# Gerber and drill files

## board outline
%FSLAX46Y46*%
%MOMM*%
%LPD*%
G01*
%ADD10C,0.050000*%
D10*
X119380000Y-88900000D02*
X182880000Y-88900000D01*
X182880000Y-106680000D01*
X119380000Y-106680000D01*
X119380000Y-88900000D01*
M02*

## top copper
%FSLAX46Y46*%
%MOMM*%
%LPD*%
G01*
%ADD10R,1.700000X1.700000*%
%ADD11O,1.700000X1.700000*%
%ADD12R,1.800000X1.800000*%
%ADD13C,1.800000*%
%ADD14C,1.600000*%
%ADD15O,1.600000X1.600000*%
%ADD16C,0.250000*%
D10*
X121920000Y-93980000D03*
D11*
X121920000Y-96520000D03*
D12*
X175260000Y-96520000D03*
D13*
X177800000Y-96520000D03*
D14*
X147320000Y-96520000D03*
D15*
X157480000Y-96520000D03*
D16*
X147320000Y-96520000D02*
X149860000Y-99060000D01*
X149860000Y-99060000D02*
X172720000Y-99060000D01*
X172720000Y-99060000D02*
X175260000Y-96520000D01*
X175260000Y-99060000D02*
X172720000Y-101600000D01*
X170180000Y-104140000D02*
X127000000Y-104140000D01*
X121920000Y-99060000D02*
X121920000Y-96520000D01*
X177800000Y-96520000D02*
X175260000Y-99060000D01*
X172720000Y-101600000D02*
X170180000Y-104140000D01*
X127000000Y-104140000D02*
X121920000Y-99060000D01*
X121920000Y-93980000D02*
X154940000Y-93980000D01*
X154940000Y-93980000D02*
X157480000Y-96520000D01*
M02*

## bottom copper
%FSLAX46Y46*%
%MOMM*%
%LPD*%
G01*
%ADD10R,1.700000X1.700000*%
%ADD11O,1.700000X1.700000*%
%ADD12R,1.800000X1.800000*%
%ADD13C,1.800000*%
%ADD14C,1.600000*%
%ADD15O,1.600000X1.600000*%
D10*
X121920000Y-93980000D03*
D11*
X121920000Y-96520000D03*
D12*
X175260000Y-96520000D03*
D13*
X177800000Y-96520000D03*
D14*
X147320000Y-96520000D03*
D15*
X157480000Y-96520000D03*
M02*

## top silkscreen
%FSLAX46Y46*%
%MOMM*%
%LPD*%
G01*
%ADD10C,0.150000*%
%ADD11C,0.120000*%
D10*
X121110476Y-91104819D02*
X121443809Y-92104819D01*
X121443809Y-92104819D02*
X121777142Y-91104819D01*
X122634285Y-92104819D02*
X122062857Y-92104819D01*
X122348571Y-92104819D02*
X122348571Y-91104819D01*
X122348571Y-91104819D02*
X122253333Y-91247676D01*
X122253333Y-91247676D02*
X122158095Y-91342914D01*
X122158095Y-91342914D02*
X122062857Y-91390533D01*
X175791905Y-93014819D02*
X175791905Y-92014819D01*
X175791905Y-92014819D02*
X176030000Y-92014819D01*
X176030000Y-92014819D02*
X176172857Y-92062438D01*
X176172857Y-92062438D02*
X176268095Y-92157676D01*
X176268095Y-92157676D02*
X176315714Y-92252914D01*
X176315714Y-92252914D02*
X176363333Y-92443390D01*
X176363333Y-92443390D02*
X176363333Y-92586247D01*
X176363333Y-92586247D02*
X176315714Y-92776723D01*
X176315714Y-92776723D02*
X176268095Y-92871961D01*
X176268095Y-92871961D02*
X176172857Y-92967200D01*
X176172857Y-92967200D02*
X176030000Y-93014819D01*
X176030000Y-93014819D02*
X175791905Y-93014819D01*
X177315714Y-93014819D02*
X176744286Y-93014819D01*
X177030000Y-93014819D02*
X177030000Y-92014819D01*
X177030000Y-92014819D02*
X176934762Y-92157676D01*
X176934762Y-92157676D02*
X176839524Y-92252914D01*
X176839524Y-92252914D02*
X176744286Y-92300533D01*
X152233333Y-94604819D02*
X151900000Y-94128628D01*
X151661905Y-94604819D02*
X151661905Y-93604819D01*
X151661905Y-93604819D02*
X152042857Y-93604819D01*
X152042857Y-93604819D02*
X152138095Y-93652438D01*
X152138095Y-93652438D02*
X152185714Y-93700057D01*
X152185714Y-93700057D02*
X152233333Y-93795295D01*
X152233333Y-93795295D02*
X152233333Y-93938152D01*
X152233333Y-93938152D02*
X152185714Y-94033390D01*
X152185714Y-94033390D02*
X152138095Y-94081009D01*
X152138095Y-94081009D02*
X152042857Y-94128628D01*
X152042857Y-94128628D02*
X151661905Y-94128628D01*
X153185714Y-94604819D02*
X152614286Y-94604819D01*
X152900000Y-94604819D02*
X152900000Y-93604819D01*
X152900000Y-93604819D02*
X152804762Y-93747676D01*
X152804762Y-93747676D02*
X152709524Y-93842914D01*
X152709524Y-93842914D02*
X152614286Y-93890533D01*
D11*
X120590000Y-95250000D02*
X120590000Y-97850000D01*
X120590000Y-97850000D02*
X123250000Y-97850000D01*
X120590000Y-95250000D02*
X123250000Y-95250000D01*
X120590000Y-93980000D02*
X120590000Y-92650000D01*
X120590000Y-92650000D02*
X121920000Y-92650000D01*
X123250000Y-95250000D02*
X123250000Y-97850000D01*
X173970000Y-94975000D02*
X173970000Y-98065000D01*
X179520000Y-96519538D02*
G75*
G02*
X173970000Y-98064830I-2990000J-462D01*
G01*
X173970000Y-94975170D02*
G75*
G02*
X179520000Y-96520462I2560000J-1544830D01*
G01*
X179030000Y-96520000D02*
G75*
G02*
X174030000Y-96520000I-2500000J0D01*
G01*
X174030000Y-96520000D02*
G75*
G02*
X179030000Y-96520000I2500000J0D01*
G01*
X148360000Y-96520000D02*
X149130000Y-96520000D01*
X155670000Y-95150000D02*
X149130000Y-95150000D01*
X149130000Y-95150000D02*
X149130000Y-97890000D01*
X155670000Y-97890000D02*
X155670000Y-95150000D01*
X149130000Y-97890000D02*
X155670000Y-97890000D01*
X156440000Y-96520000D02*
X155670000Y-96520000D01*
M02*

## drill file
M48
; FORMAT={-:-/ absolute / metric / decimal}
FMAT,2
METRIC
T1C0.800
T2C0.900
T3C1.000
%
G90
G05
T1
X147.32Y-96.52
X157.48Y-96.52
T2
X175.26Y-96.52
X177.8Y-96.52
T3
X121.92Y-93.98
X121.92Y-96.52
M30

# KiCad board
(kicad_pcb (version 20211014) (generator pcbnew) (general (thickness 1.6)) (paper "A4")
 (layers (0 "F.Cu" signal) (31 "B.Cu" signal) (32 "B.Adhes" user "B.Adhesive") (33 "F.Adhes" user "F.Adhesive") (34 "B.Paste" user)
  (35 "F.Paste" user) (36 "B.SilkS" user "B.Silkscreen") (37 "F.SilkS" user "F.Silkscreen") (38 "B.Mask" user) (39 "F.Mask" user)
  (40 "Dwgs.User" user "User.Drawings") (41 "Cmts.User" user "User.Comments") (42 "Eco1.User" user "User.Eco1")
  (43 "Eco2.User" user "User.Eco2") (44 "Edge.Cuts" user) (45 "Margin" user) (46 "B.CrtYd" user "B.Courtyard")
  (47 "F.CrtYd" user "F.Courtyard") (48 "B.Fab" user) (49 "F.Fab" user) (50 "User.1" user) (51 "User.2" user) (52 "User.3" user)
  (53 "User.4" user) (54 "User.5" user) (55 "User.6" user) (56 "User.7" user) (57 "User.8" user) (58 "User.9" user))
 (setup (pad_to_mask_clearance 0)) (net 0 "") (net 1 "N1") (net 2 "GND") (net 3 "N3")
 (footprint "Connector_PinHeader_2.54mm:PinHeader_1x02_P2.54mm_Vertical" (layer "F.Cu") (at 121.92 93.98)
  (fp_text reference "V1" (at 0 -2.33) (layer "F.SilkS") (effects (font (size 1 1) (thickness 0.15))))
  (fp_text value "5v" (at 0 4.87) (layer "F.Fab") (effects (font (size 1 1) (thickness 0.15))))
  (fp_line (start -1.33 1.27) (end -1.33 3.87) (layer "F.SilkS") (width 0.12))
  (fp_line (start -1.33 3.87) (end 1.33 3.87) (layer "F.SilkS") (width 0.12))
  (fp_line (start -1.33 1.27) (end 1.33 1.27) (layer "F.SilkS") (width 0.12))
  (fp_line (start -1.33 0) (end -1.33 -1.33) (layer "F.SilkS") (width 0.12))
  (fp_line (start -1.33 -1.33) (end 0 -1.33) (layer "F.SilkS") (width 0.12))
  (fp_line (start 1.33 1.27) (end 1.33 3.87) (layer "F.SilkS") (width 0.12))
  (pad "1" thru_hole rect (at 0 0) (size 1.7 1.7) (drill 1) (layers *.Cu *.Mask) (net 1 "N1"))
  (pad "2" thru_hole oval (at 0 2.54) (size 1.7 1.7) (drill 1) (layers *.Cu *.Mask) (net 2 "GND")))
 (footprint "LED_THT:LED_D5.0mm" (layer "F.Cu") (at 175.26 96.52)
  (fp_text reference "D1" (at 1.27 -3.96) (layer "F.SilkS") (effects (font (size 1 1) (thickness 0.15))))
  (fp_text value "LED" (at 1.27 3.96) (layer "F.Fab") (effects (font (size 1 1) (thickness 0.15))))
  (fp_line (start -1.29 -1.545) (end -1.29 1.545) (layer "F.SilkS") (width 0.12))
  (fp_arc (start 4.26 -0.000462) (mid 2.072002 2.880433) (end -1.29 1.54483) (layer "F.SilkS") (width 0.12))
  (fp_arc (start -1.29 -1.54483) (mid 2.072002 -2.880433) (end 4.26 0.000462) (layer "F.SilkS") (width 0.12))
  (fp_circle (center 1.27 0) (end 3.77 0) (layer "F.SilkS") (width 0.12) (fill none))
  (pad "1" thru_hole rect (at 0 0) (size 1.8 1.8) (drill 0.9) (layers *.Cu *.Mask) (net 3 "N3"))
  (pad "2" thru_hole circle (at 2.54 0) (size 1.8 1.8) (drill 0.9) (layers *.Cu *.Mask) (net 2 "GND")))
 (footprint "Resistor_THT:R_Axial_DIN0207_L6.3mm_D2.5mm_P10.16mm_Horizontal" (layer "F.Cu") (at 147.32 96.52)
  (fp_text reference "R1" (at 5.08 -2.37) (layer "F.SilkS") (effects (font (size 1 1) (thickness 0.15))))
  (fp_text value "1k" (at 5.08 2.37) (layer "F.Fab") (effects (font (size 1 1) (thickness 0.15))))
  (fp_line (start 1.04 0) (end 1.81 0) (layer "F.SilkS") (width 0.12))
  (fp_line (start 8.35 -1.37) (end 1.81 -1.37) (layer "F.SilkS") (width 0.12))
  (fp_line (start 1.81 -1.37) (end 1.81 1.37) (layer "F.SilkS") (width 0.12))
  (fp_line (start 8.35 1.37) (end 8.35 -1.37) (layer "F.SilkS") (width 0.12))
  (fp_line (start 1.81 1.37) (end 8.35 1.37) (layer "F.SilkS") (width 0.12))
  (fp_line (start 9.12 0) (end 8.35 0) (layer "F.SilkS") (width 0.12))
  (pad "1" thru_hole circle (at 0 0) (size 1.6 1.6) (drill 0.8) (layers *.Cu *.Mask) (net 3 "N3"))
  (pad "2" thru_hole oval (at 10.16 0) (size 1.6 1.6) (drill 0.8) (layers *.Cu *.Mask) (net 1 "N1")))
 (gr_rect (start 119.38 88.9) (end 182.88 106.68) (layer "Edge.Cuts") (width 0.05) (fill none))
 (segment (start 147.32 96.52) (end 149.86 99.06) (width 0.25) (layer "F.Cu") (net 3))
 (segment (start 149.86 99.06) (end 172.72 99.06) (width 0.25) (layer "F.Cu") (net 3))
 (segment (start 172.72 99.06) (end 175.26 96.52) (width 0.25) (layer "F.Cu") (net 3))
 (segment (start 175.26 99.06) (end 172.72 101.6) (width 0.25) (layer "F.Cu") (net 2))
 (segment (start 170.18 104.14) (end 127 104.14) (width 0.25) (layer "F.Cu") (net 2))
 (segment (start 121.92 99.06) (end 121.92 96.52) (width 0.25) (layer "F.Cu") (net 2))
 (segment (start 177.8 96.52) (end 175.26 99.06) (width 0.25) (layer "F.Cu") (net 2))
 (segment (start 172.72 101.6) (end 170.18 104.14) (width 0.25) (layer "F.Cu") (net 2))
 (segment (start 127 104.14) (end 121.92 99.06) (width 0.25) (layer "F.Cu") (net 2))
 (segment (start 121.92 93.98) (end 154.94 93.98) (width 0.25) (layer "F.Cu") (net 1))
 (segment (start 154.94 93.98) (end 157.48 96.52) (width 0.25) (layer "F.Cu") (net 1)))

